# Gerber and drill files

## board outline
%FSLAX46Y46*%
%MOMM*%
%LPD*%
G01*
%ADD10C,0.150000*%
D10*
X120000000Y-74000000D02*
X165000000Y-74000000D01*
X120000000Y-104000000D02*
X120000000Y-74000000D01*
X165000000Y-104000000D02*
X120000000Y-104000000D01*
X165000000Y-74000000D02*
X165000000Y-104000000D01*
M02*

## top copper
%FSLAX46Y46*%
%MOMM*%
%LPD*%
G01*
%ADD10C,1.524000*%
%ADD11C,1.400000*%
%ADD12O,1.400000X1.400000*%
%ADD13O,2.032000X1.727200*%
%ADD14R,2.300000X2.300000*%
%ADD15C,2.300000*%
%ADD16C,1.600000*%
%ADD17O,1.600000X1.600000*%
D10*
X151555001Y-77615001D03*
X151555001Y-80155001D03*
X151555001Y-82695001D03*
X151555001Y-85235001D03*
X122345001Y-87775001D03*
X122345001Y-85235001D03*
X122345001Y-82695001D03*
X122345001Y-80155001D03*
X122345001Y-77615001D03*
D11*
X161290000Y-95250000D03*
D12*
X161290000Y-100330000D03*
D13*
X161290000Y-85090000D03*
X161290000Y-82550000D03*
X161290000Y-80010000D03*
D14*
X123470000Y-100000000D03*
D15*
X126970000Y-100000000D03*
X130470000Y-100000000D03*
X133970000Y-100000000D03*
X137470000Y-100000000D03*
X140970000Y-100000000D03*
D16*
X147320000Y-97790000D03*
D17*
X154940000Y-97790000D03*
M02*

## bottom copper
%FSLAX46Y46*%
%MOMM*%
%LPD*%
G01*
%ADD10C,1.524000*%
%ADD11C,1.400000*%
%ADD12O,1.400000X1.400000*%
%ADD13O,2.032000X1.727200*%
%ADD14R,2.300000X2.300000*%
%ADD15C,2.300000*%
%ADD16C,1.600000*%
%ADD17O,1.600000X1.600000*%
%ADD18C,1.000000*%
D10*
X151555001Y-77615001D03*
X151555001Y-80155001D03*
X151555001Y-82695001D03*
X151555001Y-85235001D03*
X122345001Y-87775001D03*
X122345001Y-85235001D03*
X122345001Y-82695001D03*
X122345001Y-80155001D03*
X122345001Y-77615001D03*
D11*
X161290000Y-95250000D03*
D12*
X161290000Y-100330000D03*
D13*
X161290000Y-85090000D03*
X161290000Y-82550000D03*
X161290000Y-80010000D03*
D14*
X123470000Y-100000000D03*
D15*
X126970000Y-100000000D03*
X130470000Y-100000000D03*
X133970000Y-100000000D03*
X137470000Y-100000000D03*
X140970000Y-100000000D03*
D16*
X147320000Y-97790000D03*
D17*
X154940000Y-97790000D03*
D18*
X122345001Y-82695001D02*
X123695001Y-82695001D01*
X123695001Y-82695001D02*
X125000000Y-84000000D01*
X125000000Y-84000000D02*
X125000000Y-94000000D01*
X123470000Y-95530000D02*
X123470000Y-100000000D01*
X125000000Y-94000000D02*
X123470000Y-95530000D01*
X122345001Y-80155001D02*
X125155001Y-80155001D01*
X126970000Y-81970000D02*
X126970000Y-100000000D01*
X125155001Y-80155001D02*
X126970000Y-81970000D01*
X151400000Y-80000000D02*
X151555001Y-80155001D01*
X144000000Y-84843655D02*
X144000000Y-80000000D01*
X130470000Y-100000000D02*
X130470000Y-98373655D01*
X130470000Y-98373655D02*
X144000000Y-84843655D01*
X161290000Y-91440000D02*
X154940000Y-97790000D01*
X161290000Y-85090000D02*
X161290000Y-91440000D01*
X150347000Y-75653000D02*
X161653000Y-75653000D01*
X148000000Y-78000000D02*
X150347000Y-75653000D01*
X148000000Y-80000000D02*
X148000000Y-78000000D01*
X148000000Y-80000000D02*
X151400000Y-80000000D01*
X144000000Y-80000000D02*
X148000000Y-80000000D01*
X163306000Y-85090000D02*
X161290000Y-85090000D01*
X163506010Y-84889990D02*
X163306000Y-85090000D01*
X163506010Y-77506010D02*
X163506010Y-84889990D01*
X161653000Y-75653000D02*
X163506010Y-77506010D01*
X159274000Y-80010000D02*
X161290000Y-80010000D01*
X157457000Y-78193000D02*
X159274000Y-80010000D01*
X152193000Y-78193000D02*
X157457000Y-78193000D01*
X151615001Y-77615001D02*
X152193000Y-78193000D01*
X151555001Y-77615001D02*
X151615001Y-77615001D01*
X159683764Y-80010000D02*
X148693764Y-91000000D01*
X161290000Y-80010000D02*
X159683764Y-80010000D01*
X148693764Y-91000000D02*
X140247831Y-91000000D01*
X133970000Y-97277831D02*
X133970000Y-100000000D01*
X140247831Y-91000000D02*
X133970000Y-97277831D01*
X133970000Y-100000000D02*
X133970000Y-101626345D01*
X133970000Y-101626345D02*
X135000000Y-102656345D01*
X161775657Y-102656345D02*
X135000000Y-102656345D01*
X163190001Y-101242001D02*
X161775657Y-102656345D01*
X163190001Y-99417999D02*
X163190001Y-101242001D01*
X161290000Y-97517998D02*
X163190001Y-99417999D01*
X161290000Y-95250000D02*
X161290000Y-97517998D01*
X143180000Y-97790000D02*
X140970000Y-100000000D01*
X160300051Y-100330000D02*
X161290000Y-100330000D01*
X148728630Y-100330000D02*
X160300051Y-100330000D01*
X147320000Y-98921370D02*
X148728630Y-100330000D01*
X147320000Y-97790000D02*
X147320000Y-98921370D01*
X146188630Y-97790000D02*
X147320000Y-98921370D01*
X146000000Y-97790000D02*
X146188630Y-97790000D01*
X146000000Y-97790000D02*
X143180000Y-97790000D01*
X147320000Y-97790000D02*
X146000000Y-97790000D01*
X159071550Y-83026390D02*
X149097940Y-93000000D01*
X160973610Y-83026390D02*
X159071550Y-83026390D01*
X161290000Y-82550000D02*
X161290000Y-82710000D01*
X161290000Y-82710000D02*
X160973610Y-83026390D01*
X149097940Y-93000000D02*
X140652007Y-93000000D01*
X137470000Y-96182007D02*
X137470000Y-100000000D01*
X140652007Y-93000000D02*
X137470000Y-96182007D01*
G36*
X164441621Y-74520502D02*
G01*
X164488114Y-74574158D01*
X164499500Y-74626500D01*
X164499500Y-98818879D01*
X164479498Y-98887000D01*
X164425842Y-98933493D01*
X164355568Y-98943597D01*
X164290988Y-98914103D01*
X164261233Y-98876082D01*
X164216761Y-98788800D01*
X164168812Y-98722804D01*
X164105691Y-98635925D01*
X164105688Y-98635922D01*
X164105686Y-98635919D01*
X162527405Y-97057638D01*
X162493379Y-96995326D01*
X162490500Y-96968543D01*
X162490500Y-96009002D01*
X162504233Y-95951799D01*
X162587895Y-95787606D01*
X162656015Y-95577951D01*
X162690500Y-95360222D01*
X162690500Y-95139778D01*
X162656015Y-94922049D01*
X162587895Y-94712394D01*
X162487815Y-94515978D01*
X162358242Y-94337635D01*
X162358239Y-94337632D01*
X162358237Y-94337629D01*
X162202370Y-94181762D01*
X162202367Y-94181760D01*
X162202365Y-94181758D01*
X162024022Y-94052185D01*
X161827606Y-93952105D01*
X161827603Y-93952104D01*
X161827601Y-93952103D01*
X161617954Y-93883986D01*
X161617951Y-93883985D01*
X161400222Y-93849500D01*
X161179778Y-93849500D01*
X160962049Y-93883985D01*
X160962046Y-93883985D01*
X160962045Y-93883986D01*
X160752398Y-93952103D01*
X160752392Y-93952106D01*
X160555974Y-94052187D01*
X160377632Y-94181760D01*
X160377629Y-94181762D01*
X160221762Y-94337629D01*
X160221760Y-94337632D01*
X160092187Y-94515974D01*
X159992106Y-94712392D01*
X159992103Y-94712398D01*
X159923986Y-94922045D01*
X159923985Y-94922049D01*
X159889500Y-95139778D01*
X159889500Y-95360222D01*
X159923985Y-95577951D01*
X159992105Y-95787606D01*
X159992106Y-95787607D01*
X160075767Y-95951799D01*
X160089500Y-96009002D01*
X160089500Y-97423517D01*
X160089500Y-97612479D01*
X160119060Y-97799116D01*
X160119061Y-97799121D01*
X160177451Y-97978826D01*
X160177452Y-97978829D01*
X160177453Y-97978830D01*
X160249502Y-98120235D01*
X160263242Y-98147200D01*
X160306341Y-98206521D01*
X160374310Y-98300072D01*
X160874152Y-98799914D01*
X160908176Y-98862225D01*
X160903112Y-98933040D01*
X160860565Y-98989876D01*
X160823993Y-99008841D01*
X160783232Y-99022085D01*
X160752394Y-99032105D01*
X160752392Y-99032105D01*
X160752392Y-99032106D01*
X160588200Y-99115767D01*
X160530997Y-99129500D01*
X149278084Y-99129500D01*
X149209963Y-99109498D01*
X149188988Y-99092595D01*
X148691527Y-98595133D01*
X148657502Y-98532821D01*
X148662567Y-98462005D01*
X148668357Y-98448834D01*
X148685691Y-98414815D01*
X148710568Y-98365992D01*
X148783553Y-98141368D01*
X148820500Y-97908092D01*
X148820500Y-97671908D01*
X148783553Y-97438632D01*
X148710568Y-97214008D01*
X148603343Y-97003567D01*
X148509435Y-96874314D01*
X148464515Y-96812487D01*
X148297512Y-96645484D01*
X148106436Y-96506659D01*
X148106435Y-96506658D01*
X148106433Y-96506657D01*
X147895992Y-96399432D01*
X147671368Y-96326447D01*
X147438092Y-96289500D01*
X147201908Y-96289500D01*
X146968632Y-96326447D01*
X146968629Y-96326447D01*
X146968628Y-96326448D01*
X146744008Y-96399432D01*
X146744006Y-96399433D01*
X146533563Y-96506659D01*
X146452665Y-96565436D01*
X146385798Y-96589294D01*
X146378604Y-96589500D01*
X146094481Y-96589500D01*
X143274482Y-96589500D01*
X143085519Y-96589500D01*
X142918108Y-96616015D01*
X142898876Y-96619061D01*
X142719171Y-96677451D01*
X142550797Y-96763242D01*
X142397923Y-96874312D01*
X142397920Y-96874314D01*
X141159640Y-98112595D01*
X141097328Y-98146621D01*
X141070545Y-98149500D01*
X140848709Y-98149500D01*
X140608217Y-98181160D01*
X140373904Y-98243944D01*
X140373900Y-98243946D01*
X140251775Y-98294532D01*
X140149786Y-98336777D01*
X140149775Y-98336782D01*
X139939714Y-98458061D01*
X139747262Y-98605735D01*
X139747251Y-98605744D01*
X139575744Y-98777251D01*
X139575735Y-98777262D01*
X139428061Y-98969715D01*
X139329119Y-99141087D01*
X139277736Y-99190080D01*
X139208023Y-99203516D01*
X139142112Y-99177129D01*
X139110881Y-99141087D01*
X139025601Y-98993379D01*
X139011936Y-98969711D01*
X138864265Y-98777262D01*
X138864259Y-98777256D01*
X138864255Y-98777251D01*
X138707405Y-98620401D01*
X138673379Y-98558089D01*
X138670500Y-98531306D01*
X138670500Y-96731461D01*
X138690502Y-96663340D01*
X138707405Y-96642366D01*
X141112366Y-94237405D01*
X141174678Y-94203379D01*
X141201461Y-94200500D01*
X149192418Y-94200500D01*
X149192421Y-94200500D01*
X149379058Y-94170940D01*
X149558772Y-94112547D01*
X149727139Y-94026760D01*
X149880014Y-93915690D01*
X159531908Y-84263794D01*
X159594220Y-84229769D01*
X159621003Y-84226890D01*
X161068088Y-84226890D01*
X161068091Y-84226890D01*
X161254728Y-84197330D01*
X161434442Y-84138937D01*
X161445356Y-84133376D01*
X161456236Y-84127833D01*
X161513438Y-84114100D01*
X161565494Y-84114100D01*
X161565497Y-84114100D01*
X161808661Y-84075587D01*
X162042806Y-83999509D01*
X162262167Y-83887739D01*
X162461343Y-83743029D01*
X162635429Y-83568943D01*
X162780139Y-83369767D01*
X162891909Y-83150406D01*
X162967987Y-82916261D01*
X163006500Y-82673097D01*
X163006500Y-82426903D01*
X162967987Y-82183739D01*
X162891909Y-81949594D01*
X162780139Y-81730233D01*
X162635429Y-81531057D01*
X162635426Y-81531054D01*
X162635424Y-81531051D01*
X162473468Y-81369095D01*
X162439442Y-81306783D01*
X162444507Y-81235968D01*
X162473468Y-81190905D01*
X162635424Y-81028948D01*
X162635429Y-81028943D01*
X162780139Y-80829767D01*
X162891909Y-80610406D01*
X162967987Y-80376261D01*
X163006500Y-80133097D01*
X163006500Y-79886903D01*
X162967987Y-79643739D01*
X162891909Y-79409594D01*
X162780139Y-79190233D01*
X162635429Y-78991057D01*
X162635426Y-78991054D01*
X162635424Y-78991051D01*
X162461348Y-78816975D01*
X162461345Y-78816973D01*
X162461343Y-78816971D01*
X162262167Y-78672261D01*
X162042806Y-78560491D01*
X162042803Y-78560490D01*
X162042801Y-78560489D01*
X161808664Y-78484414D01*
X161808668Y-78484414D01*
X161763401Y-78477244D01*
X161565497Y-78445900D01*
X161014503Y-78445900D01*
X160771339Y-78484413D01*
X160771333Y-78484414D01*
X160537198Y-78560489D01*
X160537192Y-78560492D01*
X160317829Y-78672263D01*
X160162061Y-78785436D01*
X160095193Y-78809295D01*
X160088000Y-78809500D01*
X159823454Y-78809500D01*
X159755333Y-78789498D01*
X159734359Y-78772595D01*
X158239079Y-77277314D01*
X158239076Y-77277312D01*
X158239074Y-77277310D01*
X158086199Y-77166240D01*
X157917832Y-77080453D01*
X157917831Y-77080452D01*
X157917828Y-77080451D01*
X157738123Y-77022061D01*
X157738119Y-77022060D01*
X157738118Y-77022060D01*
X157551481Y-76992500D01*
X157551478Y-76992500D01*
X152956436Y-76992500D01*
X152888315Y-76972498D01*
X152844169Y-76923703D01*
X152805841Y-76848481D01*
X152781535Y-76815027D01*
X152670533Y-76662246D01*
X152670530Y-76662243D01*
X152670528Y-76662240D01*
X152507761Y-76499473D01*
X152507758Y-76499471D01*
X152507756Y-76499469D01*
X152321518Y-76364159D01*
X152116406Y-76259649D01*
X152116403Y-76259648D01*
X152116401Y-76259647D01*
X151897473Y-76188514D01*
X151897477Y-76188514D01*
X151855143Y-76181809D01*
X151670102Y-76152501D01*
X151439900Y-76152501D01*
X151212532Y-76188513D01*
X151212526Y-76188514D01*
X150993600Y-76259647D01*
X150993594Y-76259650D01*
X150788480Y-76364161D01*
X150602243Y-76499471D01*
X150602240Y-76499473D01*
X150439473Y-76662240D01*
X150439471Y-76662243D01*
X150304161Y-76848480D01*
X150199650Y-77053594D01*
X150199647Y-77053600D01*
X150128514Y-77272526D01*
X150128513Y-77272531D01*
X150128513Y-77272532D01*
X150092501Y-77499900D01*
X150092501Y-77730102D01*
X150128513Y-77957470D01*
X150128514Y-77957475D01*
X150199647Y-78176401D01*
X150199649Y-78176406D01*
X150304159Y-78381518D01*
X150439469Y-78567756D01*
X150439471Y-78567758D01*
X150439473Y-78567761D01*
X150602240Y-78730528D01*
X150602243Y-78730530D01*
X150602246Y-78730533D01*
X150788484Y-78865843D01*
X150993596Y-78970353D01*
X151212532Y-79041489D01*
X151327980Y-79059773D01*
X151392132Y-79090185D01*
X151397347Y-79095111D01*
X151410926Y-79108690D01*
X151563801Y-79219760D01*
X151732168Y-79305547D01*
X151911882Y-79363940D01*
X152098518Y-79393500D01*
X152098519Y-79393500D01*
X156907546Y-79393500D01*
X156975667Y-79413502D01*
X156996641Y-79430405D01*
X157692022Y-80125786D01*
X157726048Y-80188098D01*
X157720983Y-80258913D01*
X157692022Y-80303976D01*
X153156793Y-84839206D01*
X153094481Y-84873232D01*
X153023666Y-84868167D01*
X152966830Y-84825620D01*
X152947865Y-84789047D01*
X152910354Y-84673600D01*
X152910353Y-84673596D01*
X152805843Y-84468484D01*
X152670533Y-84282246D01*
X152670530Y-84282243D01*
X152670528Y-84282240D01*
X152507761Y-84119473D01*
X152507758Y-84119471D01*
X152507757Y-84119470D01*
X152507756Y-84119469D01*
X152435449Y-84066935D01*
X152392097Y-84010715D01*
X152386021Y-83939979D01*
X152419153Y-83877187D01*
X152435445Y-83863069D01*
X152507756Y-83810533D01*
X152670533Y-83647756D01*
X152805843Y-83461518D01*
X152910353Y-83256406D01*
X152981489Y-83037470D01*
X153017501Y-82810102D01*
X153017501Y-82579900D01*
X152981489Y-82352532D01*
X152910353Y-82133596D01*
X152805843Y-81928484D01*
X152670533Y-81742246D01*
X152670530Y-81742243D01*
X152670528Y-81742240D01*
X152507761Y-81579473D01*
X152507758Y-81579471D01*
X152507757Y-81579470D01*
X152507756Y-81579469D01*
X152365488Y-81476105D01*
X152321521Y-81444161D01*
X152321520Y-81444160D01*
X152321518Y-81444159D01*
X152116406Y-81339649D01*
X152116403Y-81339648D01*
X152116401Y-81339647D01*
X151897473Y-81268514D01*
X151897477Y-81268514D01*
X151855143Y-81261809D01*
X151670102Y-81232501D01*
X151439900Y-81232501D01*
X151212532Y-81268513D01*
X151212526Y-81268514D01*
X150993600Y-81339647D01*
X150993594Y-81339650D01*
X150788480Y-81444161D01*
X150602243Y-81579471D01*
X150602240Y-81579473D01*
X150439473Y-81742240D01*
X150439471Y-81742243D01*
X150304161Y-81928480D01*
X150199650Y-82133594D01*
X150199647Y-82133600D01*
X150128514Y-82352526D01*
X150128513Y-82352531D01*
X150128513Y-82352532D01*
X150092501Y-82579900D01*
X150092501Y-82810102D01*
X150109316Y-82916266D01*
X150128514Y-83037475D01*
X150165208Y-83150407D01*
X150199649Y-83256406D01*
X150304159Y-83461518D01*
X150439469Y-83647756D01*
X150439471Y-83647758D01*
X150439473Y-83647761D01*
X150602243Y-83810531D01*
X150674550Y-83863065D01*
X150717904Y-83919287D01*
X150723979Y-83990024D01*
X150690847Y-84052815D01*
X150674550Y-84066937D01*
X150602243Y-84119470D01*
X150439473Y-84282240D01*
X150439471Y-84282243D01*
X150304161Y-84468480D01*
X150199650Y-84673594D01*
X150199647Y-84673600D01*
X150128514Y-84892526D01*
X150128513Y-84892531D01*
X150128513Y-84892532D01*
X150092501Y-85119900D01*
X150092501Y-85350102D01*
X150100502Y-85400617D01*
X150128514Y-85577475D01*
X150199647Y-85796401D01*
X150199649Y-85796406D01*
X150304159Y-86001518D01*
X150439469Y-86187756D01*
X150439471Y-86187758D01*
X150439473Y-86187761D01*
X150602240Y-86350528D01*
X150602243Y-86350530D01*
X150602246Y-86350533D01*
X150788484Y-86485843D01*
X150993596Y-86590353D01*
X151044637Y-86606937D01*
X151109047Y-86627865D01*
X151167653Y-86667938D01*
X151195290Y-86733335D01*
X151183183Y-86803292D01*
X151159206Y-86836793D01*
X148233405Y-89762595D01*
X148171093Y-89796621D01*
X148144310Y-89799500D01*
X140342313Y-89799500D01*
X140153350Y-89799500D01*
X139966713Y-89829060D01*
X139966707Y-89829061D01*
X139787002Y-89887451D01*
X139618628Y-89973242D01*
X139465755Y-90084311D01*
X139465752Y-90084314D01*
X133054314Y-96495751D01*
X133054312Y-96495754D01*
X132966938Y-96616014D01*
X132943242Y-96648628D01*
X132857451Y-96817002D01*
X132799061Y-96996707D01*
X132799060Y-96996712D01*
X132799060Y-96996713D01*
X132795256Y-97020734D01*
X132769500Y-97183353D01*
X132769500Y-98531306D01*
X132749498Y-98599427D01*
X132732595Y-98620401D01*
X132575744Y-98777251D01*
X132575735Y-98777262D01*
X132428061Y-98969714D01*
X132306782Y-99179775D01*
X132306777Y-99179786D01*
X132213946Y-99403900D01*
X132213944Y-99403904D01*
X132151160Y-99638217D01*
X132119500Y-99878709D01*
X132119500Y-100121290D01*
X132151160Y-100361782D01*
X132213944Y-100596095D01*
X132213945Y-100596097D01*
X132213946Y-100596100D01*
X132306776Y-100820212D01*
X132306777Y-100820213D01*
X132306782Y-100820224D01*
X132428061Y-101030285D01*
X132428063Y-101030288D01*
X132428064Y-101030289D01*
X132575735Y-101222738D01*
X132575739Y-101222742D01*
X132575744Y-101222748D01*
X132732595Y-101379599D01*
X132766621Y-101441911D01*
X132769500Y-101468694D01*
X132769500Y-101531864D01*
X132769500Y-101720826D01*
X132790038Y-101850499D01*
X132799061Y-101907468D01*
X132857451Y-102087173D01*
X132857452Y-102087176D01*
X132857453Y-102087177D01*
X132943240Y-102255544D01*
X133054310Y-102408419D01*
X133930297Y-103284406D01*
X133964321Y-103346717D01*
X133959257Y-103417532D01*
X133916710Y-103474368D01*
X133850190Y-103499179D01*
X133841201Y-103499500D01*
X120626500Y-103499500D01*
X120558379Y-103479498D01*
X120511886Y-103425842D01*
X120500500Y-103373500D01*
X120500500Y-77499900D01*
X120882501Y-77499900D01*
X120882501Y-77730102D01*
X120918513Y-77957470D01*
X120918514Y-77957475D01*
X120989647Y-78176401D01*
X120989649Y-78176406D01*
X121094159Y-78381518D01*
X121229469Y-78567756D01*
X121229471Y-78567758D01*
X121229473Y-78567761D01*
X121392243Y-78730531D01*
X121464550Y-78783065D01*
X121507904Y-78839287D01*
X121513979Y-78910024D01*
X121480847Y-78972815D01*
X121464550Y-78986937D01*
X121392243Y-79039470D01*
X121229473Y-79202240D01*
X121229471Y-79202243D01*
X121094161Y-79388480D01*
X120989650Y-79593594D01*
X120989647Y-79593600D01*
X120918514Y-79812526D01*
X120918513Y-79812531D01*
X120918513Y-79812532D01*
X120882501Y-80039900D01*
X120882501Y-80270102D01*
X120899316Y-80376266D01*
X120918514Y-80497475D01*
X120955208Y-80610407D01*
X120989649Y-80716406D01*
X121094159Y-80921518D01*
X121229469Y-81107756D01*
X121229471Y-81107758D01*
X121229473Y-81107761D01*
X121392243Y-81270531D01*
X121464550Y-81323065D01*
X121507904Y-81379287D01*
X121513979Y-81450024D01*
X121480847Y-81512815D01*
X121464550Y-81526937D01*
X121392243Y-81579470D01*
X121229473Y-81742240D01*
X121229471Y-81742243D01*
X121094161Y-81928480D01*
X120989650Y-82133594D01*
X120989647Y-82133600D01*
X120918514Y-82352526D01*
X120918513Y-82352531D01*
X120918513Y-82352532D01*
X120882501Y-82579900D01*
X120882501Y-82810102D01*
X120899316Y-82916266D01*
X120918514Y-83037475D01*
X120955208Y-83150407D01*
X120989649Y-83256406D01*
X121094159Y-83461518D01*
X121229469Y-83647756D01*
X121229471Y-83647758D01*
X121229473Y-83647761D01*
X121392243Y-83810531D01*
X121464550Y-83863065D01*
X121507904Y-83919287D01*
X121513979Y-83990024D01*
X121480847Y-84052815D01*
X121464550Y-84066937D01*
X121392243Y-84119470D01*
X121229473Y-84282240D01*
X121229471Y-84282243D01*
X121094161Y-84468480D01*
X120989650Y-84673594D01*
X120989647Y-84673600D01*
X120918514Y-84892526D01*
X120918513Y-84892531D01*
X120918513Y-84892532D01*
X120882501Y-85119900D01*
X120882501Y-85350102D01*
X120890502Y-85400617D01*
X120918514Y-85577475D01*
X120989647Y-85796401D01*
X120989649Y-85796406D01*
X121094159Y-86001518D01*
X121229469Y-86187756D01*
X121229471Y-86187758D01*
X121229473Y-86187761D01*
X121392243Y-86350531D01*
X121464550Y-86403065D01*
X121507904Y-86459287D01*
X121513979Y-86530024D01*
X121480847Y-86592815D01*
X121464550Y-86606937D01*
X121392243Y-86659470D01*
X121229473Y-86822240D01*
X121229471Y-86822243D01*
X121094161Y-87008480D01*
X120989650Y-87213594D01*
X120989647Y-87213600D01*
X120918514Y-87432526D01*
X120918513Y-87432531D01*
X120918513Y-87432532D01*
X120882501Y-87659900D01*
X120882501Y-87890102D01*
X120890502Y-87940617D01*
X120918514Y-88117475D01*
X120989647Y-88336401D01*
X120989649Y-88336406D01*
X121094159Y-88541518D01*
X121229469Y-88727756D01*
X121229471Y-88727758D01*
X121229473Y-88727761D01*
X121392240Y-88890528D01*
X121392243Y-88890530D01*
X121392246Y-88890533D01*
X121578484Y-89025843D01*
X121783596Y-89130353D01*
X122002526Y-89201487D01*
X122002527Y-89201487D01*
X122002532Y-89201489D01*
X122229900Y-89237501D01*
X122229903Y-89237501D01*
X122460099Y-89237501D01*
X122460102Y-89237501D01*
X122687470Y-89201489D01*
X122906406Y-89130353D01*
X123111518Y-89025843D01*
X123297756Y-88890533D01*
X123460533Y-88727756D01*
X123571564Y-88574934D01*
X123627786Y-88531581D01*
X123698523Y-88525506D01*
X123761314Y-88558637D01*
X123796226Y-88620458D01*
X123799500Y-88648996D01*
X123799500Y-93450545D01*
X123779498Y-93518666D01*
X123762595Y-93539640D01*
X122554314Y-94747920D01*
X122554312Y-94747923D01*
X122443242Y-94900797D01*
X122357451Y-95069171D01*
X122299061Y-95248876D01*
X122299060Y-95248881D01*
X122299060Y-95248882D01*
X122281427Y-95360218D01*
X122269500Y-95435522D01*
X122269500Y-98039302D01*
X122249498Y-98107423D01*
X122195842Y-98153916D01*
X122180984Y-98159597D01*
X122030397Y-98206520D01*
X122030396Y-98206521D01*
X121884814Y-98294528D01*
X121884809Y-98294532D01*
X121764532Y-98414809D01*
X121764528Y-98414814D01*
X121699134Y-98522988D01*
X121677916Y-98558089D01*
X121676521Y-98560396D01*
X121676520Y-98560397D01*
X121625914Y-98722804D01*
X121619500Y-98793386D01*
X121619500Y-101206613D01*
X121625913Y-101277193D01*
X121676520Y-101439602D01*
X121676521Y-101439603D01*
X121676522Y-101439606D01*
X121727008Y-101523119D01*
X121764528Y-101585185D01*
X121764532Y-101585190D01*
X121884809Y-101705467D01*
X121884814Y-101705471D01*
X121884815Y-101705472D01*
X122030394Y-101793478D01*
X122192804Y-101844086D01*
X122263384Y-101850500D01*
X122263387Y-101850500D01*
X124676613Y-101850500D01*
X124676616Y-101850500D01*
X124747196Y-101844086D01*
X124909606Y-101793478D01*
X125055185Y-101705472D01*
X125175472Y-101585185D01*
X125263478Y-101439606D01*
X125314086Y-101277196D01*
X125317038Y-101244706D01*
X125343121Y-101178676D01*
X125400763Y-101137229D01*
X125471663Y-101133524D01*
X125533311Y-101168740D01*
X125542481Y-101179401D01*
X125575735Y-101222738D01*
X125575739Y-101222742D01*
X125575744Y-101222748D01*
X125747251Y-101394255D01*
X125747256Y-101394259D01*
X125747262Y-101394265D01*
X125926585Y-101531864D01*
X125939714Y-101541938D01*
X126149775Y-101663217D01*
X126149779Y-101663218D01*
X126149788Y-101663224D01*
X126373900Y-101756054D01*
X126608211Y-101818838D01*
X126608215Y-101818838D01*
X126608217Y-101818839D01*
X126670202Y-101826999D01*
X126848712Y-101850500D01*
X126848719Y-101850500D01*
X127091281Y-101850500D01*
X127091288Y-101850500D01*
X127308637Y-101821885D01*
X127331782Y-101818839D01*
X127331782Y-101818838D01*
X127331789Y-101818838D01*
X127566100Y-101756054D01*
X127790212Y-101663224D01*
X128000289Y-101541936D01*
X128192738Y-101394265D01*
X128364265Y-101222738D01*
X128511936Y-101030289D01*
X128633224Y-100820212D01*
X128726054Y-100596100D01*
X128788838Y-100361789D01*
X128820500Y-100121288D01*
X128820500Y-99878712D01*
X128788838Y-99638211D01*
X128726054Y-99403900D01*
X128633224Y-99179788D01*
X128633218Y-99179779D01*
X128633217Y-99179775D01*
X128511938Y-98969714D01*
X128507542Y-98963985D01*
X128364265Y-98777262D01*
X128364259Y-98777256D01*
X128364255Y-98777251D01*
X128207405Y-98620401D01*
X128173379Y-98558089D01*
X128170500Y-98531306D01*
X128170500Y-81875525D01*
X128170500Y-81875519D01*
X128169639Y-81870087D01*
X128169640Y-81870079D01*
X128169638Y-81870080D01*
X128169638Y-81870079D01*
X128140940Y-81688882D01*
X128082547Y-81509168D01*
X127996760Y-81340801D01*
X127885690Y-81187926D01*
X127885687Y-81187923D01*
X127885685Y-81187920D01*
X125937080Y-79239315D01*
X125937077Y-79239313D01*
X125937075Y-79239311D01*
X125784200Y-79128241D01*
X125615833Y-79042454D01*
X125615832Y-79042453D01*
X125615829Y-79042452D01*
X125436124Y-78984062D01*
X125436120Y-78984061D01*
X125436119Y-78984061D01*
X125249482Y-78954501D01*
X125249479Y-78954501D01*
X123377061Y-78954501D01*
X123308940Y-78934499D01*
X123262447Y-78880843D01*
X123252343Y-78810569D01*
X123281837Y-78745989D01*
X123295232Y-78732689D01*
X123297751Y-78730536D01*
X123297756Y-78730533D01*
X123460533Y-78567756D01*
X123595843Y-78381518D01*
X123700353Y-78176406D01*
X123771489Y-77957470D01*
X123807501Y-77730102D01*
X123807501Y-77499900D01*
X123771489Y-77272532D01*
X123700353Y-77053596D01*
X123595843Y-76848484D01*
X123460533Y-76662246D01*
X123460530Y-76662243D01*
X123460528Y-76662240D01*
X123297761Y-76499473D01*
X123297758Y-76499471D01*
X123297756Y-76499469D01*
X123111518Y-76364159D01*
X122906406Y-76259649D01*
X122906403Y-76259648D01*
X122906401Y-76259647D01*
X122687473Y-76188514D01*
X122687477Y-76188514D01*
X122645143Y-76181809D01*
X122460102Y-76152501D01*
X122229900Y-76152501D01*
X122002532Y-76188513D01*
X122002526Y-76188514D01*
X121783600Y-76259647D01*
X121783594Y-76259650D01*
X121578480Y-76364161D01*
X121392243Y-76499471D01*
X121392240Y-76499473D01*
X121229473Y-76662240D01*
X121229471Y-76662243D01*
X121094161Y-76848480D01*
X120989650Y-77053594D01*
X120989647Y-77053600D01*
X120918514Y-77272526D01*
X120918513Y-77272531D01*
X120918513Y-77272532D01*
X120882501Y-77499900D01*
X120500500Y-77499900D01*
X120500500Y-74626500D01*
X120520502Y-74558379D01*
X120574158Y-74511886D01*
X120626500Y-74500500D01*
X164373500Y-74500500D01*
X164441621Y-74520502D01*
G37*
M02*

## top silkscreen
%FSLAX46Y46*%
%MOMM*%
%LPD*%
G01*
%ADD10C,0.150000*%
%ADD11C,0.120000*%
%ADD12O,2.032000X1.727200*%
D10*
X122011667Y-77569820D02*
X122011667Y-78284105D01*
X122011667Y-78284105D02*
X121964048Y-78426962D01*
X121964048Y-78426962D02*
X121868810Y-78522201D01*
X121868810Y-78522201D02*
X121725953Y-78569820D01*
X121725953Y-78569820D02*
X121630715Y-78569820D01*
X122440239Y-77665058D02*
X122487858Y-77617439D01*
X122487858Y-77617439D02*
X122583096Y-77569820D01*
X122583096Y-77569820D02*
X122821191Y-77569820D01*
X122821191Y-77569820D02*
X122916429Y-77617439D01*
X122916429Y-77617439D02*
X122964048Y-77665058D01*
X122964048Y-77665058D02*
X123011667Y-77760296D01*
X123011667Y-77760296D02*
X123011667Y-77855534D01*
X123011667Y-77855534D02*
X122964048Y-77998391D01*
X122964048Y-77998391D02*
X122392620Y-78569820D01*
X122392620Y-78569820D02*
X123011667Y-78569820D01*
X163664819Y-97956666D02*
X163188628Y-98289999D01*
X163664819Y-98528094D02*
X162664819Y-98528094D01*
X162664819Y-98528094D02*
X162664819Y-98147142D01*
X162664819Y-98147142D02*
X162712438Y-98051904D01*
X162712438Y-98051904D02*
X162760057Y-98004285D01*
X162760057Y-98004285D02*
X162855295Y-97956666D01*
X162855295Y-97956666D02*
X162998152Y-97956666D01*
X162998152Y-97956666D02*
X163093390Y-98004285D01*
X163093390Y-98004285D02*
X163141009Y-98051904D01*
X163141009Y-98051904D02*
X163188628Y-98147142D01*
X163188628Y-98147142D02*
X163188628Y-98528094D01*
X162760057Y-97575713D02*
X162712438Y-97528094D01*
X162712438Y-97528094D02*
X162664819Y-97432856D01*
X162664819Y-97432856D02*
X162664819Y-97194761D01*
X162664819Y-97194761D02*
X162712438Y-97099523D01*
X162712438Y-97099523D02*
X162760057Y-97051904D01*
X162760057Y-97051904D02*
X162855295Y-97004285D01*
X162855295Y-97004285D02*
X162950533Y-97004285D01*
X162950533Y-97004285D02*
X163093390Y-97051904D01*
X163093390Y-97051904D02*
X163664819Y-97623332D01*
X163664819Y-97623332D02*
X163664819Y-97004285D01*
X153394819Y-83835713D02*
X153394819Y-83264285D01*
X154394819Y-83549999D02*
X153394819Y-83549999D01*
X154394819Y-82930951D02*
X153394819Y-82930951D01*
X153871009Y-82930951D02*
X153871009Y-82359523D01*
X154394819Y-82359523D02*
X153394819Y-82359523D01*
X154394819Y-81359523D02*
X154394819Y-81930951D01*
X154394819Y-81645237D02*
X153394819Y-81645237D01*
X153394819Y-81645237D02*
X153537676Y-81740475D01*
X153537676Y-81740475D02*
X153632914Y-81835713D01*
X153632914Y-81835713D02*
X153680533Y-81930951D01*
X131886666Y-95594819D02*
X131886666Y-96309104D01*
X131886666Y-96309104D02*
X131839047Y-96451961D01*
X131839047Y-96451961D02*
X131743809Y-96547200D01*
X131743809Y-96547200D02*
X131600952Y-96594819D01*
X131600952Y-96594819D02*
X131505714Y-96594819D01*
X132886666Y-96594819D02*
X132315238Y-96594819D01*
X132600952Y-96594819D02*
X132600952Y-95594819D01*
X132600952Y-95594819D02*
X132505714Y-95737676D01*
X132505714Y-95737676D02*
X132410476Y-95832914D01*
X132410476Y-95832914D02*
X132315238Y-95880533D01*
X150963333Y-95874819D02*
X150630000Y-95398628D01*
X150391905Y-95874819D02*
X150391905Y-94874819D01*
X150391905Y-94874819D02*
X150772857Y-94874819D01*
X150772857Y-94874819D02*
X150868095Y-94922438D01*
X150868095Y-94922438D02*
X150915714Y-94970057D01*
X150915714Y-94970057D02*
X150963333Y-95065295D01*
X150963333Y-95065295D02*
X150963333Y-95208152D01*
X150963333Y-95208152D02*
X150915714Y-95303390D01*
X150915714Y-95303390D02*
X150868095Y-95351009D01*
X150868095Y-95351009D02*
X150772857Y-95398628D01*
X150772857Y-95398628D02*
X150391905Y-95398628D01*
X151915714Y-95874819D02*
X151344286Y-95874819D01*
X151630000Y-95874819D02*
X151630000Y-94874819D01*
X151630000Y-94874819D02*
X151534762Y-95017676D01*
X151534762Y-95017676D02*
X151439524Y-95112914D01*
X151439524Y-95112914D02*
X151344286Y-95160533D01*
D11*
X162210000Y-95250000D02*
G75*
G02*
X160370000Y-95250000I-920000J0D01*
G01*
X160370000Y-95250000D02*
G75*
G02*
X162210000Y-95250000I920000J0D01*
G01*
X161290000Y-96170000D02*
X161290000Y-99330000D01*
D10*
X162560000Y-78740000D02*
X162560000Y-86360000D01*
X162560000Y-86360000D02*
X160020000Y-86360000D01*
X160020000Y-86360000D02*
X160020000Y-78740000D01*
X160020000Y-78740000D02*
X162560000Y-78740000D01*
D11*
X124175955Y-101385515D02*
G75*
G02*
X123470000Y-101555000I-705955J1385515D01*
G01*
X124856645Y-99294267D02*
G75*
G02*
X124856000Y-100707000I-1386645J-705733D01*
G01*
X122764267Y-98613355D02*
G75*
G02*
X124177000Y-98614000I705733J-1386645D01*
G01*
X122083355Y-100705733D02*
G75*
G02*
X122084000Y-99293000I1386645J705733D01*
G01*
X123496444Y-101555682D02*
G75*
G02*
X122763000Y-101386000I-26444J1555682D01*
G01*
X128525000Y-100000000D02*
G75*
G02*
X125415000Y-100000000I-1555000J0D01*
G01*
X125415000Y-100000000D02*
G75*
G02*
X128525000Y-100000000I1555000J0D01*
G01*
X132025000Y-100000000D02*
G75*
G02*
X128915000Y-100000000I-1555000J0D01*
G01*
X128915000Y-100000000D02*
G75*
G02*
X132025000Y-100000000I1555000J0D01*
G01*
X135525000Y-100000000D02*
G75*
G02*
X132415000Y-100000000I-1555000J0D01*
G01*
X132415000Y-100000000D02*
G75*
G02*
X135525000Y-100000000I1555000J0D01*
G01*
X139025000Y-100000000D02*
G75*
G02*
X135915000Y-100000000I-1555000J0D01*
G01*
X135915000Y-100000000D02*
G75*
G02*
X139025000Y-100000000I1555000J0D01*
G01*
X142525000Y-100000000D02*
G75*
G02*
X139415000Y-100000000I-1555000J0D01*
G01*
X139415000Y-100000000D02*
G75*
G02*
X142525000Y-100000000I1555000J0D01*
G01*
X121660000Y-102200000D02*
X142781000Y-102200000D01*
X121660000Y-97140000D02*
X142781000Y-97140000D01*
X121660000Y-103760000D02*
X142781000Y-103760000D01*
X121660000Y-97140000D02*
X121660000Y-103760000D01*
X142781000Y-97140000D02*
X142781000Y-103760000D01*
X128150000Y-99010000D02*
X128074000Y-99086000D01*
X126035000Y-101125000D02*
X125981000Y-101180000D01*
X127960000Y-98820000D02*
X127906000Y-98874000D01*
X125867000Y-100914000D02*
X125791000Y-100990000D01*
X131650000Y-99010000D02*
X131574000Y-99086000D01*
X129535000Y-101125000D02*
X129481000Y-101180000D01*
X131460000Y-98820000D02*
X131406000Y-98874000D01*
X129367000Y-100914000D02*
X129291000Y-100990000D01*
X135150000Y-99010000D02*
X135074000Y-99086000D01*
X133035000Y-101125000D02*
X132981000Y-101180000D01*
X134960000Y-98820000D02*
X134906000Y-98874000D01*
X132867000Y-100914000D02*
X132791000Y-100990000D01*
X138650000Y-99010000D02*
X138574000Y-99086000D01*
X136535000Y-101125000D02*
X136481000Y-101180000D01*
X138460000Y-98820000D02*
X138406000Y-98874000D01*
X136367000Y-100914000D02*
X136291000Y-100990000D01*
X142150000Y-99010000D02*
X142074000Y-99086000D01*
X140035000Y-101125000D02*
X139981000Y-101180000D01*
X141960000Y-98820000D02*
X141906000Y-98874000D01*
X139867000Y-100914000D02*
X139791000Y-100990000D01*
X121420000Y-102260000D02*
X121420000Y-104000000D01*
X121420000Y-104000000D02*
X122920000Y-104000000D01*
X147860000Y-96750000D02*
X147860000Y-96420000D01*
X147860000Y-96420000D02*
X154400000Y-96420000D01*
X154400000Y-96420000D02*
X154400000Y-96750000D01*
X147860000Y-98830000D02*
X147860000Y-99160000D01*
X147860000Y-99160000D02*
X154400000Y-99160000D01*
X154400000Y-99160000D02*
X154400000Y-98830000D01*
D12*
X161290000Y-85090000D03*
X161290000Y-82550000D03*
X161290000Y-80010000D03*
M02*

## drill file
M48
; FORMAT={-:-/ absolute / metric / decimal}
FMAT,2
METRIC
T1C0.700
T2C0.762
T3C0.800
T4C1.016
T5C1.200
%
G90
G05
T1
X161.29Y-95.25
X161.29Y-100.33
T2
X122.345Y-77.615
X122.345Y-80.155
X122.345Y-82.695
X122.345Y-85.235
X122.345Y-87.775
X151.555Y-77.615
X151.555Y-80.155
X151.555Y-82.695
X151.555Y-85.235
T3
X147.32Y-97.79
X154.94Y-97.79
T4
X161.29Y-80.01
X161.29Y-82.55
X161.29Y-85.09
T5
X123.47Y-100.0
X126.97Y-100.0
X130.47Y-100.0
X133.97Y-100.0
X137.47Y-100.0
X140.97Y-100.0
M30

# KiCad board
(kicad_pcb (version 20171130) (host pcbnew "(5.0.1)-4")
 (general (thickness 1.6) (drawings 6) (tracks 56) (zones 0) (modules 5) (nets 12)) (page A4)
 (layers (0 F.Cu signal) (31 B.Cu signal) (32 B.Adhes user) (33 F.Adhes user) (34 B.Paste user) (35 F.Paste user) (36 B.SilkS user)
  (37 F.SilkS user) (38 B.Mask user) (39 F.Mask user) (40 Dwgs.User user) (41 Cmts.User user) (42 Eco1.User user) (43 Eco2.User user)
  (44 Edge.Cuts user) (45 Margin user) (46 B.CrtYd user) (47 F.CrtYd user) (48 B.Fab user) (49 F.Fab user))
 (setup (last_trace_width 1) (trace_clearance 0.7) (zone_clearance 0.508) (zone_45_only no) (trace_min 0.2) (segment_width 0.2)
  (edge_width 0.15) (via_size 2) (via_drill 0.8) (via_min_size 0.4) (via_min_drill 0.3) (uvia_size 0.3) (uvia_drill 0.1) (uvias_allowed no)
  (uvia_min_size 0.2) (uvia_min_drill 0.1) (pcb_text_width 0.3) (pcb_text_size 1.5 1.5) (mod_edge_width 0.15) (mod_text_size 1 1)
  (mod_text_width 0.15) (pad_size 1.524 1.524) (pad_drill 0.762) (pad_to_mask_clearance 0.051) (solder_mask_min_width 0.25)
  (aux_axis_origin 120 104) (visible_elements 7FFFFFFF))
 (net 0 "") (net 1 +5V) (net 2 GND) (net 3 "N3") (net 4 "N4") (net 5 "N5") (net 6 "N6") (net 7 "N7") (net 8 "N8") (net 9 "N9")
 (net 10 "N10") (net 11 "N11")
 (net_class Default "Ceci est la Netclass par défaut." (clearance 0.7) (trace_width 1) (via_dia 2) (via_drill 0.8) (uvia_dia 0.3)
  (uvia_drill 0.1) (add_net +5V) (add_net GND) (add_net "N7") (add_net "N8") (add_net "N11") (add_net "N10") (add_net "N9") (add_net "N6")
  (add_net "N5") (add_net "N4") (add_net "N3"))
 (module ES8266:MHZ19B (layer F.Cu) (at 122.345001 77.615001)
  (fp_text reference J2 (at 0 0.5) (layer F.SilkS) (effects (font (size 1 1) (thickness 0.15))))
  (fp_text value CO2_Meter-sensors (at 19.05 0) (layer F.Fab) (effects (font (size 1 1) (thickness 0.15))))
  (pad 9 thru_hole circle (at 29.21 0) (size 1.524 1.524) (drill 0.762) (layers *.Cu *.Mask) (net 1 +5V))
  (pad 8 thru_hole circle (at 29.21 2.54) (size 1.524 1.524) (drill 0.762) (layers *.Cu *.Mask) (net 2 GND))
  (pad 7 thru_hole circle (at 29.21 5.08) (size 1.524 1.524) (drill 0.762) (layers *.Cu *.Mask) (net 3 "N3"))
  (pad 6 thru_hole circle (at 29.21 7.62) (size 1.524 1.524) (drill 0.762) (layers *.Cu *.Mask) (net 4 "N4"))
  (pad 5 thru_hole circle (at 0 10.16) (size 1.524 1.524) (drill 0.762) (layers *.Cu *.Mask) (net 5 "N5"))
  (pad 4 thru_hole circle (at 0 7.62) (size 1.524 1.524) (drill 0.762) (layers *.Cu *.Mask) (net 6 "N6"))
  (pad 3 thru_hole circle (at 0 5.08) (size 1.524 1.524) (drill 0.762) (layers *.Cu *.Mask) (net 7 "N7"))
  (pad 2 thru_hole circle (at 0 2.54) (size 1.524 1.524) (drill 0.762) (layers *.Cu *.Mask) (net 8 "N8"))
  (pad 1 thru_hole circle (at 0 0) (size 1.524 1.524) (drill 0.762) (layers *.Cu *.Mask) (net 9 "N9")))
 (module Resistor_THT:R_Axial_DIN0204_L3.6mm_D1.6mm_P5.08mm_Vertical (layer F.Cu) (at 161.29 95.25 270)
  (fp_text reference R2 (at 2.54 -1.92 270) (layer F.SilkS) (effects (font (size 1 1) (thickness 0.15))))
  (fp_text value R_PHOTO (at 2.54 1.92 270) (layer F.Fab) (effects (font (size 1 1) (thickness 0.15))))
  (fp_circle (center 0 0) (end 0.92 0) (layer F.SilkS) (width 0.12))
  (fp_line (start 0.92 0) (end 4.08 0) (layer F.SilkS) (width 0.12))
  (pad 1 thru_hole circle (at 0 0 270) (size 1.4 1.4) (drill 0.7) (layers *.Cu *.Mask) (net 1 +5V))
  (pad 2 thru_hole oval (at 5.08 0 270) (size 1.4 1.4) (drill 0.7) (layers *.Cu *.Mask) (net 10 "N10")))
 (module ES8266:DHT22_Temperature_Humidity (layer F.Cu) (at 161.29 82.55 270)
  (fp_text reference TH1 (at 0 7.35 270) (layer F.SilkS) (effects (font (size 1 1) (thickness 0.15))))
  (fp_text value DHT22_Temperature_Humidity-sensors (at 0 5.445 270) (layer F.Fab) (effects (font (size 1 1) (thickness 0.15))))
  (fp_line (start -3.81 -1.27) (end 3.81 -1.27) (layer F.SilkS) (width 0.15))
  (fp_line (start 3.81 -1.27) (end 3.81 1.27) (layer F.SilkS) (width 0.15))
  (fp_line (start 3.81 1.27) (end -3.81 1.27) (layer F.SilkS) (width 0.15))
  (fp_line (start -3.81 1.27) (end -3.81 -1.27) (layer F.SilkS) (width 0.15))
  (pad 3 thru_hole oval (at 2.54 0) (size 2.032 1.7272) (drill 1.016) (layers *.Cu *.Mask F.SilkS) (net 2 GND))
  (pad 2 thru_hole oval (at 0 0) (size 2.032 1.7272) (drill 1.016) (layers *.Cu *.Mask F.SilkS) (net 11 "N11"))
  (pad 1 thru_hole oval (at -2.54 0) (size 2.032 1.7272) (drill 1.016) (layers *.Cu *.Mask F.SilkS) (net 1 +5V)))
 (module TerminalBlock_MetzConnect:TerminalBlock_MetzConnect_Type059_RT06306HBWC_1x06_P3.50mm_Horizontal (layer F.Cu) (at 123.47 100)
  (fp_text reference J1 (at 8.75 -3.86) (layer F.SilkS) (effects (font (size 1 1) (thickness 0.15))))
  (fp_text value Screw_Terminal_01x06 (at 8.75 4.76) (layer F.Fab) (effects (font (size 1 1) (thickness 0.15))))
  (fp_arc (start 0 0) (end 0 1.555) (angle -27) (layer F.SilkS) (width 0.12))
  (fp_arc (start 0 0) (end 1.386 0.707) (angle -54) (layer F.SilkS) (width 0.12))
  (fp_arc (start 0 0) (end 0.707 -1.386) (angle -54) (layer F.SilkS) (width 0.12))
  (fp_arc (start 0 0) (end -1.386 -0.707) (angle -54) (layer F.SilkS) (width 0.12))
  (fp_arc (start 0 0) (end -0.707 1.386) (angle -28) (layer F.SilkS) (width 0.12))
  (fp_circle (center 3.5 0) (end 5.055 0) (layer F.SilkS) (width 0.12))
  (fp_circle (center 7 0) (end 8.555 0) (layer F.SilkS) (width 0.12))
  (fp_circle (center 10.5 0) (end 12.055 0) (layer F.SilkS) (width 0.12))
  (fp_circle (center 14 0) (end 15.555 0) (layer F.SilkS) (width 0.12))
  (fp_circle (center 17.5 0) (end 19.055 0) (layer F.SilkS) (width 0.12))
  (fp_line (start -1.81 2.2) (end 19.311 2.2) (layer F.SilkS) (width 0.12))
  (fp_line (start -1.81 -2.86) (end 19.311 -2.86) (layer F.SilkS) (width 0.12))
  (fp_line (start -1.81 3.76) (end 19.311 3.76) (layer F.SilkS) (width 0.12))
  (fp_line (start -1.81 -2.86) (end -1.81 3.76) (layer F.SilkS) (width 0.12))
  (fp_line (start 19.311 -2.86) (end 19.311 3.76) (layer F.SilkS) (width 0.12))
  (fp_line (start 4.68 -0.99) (end 4.604 -0.914) (layer F.SilkS) (width 0.12))
  (fp_line (start 2.565 1.125) (end 2.511 1.18) (layer F.SilkS) (width 0.12))
  (fp_line (start 4.49 -1.18) (end 4.436 -1.126) (layer F.SilkS) (width 0.12))
  (fp_line (start 2.397 0.914) (end 2.321 0.99) (layer F.SilkS) (width 0.12))
  (fp_line (start 8.18 -0.99) (end 8.104 -0.914) (layer F.SilkS) (width 0.12))
  (fp_line (start 6.065 1.125) (end 6.011 1.18) (layer F.SilkS) (width 0.12))
  (fp_line (start 7.99 -1.18) (end 7.936 -1.126) (layer F.SilkS) (width 0.12))
  (fp_line (start 5.897 0.914) (end 5.821 0.99) (layer F.SilkS) (width 0.12))
  (fp_line (start 11.68 -0.99) (end 11.604 -0.914) (layer F.SilkS) (width 0.12))
  (fp_line (start 9.565 1.125) (end 9.511 1.18) (layer F.SilkS) (width 0.12))
  (fp_line (start 11.49 -1.18) (end 11.436 -1.126) (layer F.SilkS) (width 0.12))
  (fp_line (start 9.397 0.914) (end 9.321 0.99) (layer F.SilkS) (width 0.12))
  (fp_line (start 15.18 -0.99) (end 15.104 -0.914) (layer F.SilkS) (width 0.12))
  (fp_line (start 13.065 1.125) (end 13.011 1.18) (layer F.SilkS) (width 0.12))
  (fp_line (start 14.99 -1.18) (end 14.936 -1.126) (layer F.SilkS) (width 0.12))
  (fp_line (start 12.897 0.914) (end 12.821 0.99) (layer F.SilkS) (width 0.12))
  (fp_line (start 18.68 -0.99) (end 18.604 -0.914) (layer F.SilkS) (width 0.12))
  (fp_line (start 16.565 1.125) (end 16.511 1.18) (layer F.SilkS) (width 0.12))
  (fp_line (start 18.49 -1.18) (end 18.436 -1.126) (layer F.SilkS) (width 0.12))
  (fp_line (start 16.397 0.914) (end 16.321 0.99) (layer F.SilkS) (width 0.12))
  (fp_line (start -2.05 2.26) (end -2.05 4) (layer F.SilkS) (width 0.12))
  (fp_line (start -2.05 4) (end -0.55 4) (layer F.SilkS) (width 0.12))
  (pad 1 thru_hole rect (at 0 0) (size 2.3 2.3) (drill 1.2) (layers *.Cu *.Mask) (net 7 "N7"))
  (pad 2 thru_hole circle (at 3.5 0) (size 2.3 2.3) (drill 1.2) (layers *.Cu *.Mask) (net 8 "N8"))
  (pad 3 thru_hole circle (at 7 0) (size 2.3 2.3) (drill 1.2) (layers *.Cu *.Mask) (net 2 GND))
  (pad 4 thru_hole circle (at 10.5 0) (size 2.3 2.3) (drill 1.2) (layers *.Cu *.Mask) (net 1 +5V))
  (pad 5 thru_hole circle (at 14 0) (size 2.3 2.3) (drill 1.2) (layers *.Cu *.Mask) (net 11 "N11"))
  (pad 6 thru_hole circle (at 17.5 0) (size 2.3 2.3) (drill 1.2) (layers *.Cu *.Mask) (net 10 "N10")))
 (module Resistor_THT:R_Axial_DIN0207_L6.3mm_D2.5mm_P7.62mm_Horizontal (layer F.Cu) (at 147.32 97.79)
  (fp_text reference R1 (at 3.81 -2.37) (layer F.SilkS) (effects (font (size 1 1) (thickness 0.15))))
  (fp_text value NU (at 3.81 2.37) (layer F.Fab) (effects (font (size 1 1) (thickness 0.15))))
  (fp_line (start 0.54 -1.04) (end 0.54 -1.37) (layer F.SilkS) (width 0.12))
  (fp_line (start 0.54 -1.37) (end 7.08 -1.37) (layer F.SilkS) (width 0.12))
  (fp_line (start 7.08 -1.37) (end 7.08 -1.04) (layer F.SilkS) (width 0.12))
  (fp_line (start 0.54 1.04) (end 0.54 1.37) (layer F.SilkS) (width 0.12))
  (fp_line (start 0.54 1.37) (end 7.08 1.37) (layer F.SilkS) (width 0.12))
  (fp_line (start 7.08 1.37) (end 7.08 1.04) (layer F.SilkS) (width 0.12))
  (pad 1 thru_hole circle (at 0 0) (size 1.6 1.6) (drill 0.8) (layers *.Cu *.Mask) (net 10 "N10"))
  (pad 2 thru_hole oval (at 7.62 0) (size 1.6 1.6) (drill 0.8) (layers *.Cu *.Mask) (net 2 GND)))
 (gr_line (start 120 74) (end 165 74) (layer Edge.Cuts) (width 0.15))
 (gr_line (start 120 104) (end 120 74) (layer Edge.Cuts) (width 0.15))
 (gr_line (start 165 104) (end 120 104) (layer Edge.Cuts) (width 0.15))
 (gr_line (start 165 74) (end 165 104) (layer Edge.Cuts) (width 0.15))
 (segment (start 122.345001 82.695001) (end 123.695001 82.695001) (width 1) (layer B.Cu) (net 7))
 (segment (start 123.695001 82.695001) (end 125 84) (width 1) (layer B.Cu) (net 7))
 (segment (start 125 84) (end 125 94) (width 1) (layer B.Cu) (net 7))
 (segment (start 123.47 95.53) (end 123.47 100) (width 1) (layer B.Cu) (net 7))
 (segment (start 125 94) (end 123.47 95.53) (width 1) (layer B.Cu) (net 7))
 (segment (start 122.345001 80.155001) (end 125.155001 80.155001) (width 1) (layer B.Cu) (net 8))
 (segment (start 126.97 81.97) (end 126.97 100) (width 1) (layer B.Cu) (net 8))
 (segment (start 125.155001 80.155001) (end 126.97 81.97) (width 1) (layer B.Cu) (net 8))
 (segment (start 151.4 80) (end 151.555001 80.155001) (width 1) (layer B.Cu) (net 2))
 (segment (start 144 84.843655) (end 144 80) (width 1) (layer B.Cu) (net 2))
 (segment (start 130.47 100) (end 130.47 98.373655) (width 1) (layer B.Cu) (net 2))
 (segment (start 130.47 98.373655) (end 144 84.843655) (width 1) (layer B.Cu) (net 2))
 (segment (start 161.29 91.44) (end 154.94 97.79) (width 1) (layer B.Cu) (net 2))
 (segment (start 161.29 85.09) (end 161.29 91.44) (width 1) (layer B.Cu) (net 2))
 (segment (start 150.347 75.653) (end 161.653 75.653) (width 1) (layer B.Cu) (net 2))
 (segment (start 148 78) (end 150.347 75.653) (width 1) (layer B.Cu) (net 2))
 (segment (start 148 80) (end 148 78) (width 1) (layer B.Cu) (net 2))
 (segment (start 148 80) (end 151.4 80) (width 1) (layer B.Cu) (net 2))
 (segment (start 144 80) (end 148 80) (width 1) (layer B.Cu) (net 2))
 (segment (start 163.306 85.09) (end 161.29 85.09) (width 1) (layer B.Cu) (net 2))
 (segment (start 163.50601 84.88999) (end 163.306 85.09) (width 1) (layer B.Cu) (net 2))
 (segment (start 163.50601 77.50601) (end 163.50601 84.88999) (width 1) (layer B.Cu) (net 2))
 (segment (start 161.653 75.653) (end 163.50601 77.50601) (width 1) (layer B.Cu) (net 2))
 (segment (start 159.274 80.01) (end 161.29 80.01) (width 1) (layer B.Cu) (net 1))
 (segment (start 157.457 78.193) (end 159.274 80.01) (width 1) (layer B.Cu) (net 1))
 (segment (start 152.193 78.193) (end 157.457 78.193) (width 1) (layer B.Cu) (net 1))
 (segment (start 151.615001 77.615001) (end 152.193 78.193) (width 1) (layer B.Cu) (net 1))
 (segment (start 151.555001 77.615001) (end 151.615001 77.615001) (width 1) (layer B.Cu) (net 1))
 (segment (start 159.683764 80.01) (end 148.693764 91) (width 1) (layer B.Cu) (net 1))
 (segment (start 161.29 80.01) (end 159.683764 80.01) (width 1) (layer B.Cu) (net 1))
 (segment (start 148.693764 91) (end 140.247831 91) (width 1) (layer B.Cu) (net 1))
 (segment (start 133.97 97.277831) (end 133.97 100) (width 1) (layer B.Cu) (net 1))
 (segment (start 140.247831 91) (end 133.97 97.277831) (width 1) (layer B.Cu) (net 1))
 (segment (start 133.97 100) (end 133.97 101.626345) (width 1) (layer B.Cu) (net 1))
 (segment (start 133.97 101.626345) (end 135 102.656345) (width 1) (layer B.Cu) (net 1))
 (segment (start 161.775657 102.656345) (end 135 102.656345) (width 1) (layer B.Cu) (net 1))
 (segment (start 163.190001 101.242001) (end 161.775657 102.656345) (width 1) (layer B.Cu) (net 1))
 (segment (start 163.190001 99.417999) (end 163.190001 101.242001) (width 1) (layer B.Cu) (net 1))
 (segment (start 161.29 97.517998) (end 163.190001 99.417999) (width 1) (layer B.Cu) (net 1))
 (segment (start 161.29 95.25) (end 161.29 97.517998) (width 1) (layer B.Cu) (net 1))
 (segment (start 143.18 97.79) (end 140.97 100) (width 1) (layer B.Cu) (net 10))
 (segment (start 160.300051 100.33) (end 161.29 100.33) (width 1) (layer B.Cu) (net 10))
 (segment (start 148.72863 100.33) (end 160.300051 100.33) (width 1) (layer B.Cu) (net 10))
 (segment (start 147.32 98.92137) (end 148.72863 100.33) (width 1) (layer B.Cu) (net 10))
 (segment (start 147.32 97.79) (end 147.32 98.92137) (width 1) (layer B.Cu) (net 10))
 (segment (start 146.18863 97.79) (end 147.32 98.92137) (width 1) (layer B.Cu) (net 10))
 (segment (start 146 97.79) (end 146.18863 97.79) (width 1) (layer B.Cu) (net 10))
 (segment (start 146 97.79) (end 143.18 97.79) (width 1) (layer B.Cu) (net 10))
 (segment (start 147.32 97.79) (end 146 97.79) (width 1) (layer B.Cu) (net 10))
 (segment (start 159.07155 83.02639) (end 149.09794 93) (width 1) (layer B.Cu) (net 11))
 (segment (start 160.97361 83.02639) (end 159.07155 83.02639) (width 1) (layer B.Cu) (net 11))
 (segment (start 161.29 82.55) (end 161.29 82.71) (width 1) (layer B.Cu) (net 11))
 (segment (start 161.29 82.71) (end 160.97361 83.02639) (width 1) (layer B.Cu) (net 11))
 (segment (start 149.09794 93) (end 140.652007 93) (width 1) (layer B.Cu) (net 11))
 (segment (start 137.47 96.182007) (end 137.47 100) (width 1) (layer B.Cu) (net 11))
 (segment (start 140.652007 93) (end 137.47 96.182007) (width 1) (layer B.Cu) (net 11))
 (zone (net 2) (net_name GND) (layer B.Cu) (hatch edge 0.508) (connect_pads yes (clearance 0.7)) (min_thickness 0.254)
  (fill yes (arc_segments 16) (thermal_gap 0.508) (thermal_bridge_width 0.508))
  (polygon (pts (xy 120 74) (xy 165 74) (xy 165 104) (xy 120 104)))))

